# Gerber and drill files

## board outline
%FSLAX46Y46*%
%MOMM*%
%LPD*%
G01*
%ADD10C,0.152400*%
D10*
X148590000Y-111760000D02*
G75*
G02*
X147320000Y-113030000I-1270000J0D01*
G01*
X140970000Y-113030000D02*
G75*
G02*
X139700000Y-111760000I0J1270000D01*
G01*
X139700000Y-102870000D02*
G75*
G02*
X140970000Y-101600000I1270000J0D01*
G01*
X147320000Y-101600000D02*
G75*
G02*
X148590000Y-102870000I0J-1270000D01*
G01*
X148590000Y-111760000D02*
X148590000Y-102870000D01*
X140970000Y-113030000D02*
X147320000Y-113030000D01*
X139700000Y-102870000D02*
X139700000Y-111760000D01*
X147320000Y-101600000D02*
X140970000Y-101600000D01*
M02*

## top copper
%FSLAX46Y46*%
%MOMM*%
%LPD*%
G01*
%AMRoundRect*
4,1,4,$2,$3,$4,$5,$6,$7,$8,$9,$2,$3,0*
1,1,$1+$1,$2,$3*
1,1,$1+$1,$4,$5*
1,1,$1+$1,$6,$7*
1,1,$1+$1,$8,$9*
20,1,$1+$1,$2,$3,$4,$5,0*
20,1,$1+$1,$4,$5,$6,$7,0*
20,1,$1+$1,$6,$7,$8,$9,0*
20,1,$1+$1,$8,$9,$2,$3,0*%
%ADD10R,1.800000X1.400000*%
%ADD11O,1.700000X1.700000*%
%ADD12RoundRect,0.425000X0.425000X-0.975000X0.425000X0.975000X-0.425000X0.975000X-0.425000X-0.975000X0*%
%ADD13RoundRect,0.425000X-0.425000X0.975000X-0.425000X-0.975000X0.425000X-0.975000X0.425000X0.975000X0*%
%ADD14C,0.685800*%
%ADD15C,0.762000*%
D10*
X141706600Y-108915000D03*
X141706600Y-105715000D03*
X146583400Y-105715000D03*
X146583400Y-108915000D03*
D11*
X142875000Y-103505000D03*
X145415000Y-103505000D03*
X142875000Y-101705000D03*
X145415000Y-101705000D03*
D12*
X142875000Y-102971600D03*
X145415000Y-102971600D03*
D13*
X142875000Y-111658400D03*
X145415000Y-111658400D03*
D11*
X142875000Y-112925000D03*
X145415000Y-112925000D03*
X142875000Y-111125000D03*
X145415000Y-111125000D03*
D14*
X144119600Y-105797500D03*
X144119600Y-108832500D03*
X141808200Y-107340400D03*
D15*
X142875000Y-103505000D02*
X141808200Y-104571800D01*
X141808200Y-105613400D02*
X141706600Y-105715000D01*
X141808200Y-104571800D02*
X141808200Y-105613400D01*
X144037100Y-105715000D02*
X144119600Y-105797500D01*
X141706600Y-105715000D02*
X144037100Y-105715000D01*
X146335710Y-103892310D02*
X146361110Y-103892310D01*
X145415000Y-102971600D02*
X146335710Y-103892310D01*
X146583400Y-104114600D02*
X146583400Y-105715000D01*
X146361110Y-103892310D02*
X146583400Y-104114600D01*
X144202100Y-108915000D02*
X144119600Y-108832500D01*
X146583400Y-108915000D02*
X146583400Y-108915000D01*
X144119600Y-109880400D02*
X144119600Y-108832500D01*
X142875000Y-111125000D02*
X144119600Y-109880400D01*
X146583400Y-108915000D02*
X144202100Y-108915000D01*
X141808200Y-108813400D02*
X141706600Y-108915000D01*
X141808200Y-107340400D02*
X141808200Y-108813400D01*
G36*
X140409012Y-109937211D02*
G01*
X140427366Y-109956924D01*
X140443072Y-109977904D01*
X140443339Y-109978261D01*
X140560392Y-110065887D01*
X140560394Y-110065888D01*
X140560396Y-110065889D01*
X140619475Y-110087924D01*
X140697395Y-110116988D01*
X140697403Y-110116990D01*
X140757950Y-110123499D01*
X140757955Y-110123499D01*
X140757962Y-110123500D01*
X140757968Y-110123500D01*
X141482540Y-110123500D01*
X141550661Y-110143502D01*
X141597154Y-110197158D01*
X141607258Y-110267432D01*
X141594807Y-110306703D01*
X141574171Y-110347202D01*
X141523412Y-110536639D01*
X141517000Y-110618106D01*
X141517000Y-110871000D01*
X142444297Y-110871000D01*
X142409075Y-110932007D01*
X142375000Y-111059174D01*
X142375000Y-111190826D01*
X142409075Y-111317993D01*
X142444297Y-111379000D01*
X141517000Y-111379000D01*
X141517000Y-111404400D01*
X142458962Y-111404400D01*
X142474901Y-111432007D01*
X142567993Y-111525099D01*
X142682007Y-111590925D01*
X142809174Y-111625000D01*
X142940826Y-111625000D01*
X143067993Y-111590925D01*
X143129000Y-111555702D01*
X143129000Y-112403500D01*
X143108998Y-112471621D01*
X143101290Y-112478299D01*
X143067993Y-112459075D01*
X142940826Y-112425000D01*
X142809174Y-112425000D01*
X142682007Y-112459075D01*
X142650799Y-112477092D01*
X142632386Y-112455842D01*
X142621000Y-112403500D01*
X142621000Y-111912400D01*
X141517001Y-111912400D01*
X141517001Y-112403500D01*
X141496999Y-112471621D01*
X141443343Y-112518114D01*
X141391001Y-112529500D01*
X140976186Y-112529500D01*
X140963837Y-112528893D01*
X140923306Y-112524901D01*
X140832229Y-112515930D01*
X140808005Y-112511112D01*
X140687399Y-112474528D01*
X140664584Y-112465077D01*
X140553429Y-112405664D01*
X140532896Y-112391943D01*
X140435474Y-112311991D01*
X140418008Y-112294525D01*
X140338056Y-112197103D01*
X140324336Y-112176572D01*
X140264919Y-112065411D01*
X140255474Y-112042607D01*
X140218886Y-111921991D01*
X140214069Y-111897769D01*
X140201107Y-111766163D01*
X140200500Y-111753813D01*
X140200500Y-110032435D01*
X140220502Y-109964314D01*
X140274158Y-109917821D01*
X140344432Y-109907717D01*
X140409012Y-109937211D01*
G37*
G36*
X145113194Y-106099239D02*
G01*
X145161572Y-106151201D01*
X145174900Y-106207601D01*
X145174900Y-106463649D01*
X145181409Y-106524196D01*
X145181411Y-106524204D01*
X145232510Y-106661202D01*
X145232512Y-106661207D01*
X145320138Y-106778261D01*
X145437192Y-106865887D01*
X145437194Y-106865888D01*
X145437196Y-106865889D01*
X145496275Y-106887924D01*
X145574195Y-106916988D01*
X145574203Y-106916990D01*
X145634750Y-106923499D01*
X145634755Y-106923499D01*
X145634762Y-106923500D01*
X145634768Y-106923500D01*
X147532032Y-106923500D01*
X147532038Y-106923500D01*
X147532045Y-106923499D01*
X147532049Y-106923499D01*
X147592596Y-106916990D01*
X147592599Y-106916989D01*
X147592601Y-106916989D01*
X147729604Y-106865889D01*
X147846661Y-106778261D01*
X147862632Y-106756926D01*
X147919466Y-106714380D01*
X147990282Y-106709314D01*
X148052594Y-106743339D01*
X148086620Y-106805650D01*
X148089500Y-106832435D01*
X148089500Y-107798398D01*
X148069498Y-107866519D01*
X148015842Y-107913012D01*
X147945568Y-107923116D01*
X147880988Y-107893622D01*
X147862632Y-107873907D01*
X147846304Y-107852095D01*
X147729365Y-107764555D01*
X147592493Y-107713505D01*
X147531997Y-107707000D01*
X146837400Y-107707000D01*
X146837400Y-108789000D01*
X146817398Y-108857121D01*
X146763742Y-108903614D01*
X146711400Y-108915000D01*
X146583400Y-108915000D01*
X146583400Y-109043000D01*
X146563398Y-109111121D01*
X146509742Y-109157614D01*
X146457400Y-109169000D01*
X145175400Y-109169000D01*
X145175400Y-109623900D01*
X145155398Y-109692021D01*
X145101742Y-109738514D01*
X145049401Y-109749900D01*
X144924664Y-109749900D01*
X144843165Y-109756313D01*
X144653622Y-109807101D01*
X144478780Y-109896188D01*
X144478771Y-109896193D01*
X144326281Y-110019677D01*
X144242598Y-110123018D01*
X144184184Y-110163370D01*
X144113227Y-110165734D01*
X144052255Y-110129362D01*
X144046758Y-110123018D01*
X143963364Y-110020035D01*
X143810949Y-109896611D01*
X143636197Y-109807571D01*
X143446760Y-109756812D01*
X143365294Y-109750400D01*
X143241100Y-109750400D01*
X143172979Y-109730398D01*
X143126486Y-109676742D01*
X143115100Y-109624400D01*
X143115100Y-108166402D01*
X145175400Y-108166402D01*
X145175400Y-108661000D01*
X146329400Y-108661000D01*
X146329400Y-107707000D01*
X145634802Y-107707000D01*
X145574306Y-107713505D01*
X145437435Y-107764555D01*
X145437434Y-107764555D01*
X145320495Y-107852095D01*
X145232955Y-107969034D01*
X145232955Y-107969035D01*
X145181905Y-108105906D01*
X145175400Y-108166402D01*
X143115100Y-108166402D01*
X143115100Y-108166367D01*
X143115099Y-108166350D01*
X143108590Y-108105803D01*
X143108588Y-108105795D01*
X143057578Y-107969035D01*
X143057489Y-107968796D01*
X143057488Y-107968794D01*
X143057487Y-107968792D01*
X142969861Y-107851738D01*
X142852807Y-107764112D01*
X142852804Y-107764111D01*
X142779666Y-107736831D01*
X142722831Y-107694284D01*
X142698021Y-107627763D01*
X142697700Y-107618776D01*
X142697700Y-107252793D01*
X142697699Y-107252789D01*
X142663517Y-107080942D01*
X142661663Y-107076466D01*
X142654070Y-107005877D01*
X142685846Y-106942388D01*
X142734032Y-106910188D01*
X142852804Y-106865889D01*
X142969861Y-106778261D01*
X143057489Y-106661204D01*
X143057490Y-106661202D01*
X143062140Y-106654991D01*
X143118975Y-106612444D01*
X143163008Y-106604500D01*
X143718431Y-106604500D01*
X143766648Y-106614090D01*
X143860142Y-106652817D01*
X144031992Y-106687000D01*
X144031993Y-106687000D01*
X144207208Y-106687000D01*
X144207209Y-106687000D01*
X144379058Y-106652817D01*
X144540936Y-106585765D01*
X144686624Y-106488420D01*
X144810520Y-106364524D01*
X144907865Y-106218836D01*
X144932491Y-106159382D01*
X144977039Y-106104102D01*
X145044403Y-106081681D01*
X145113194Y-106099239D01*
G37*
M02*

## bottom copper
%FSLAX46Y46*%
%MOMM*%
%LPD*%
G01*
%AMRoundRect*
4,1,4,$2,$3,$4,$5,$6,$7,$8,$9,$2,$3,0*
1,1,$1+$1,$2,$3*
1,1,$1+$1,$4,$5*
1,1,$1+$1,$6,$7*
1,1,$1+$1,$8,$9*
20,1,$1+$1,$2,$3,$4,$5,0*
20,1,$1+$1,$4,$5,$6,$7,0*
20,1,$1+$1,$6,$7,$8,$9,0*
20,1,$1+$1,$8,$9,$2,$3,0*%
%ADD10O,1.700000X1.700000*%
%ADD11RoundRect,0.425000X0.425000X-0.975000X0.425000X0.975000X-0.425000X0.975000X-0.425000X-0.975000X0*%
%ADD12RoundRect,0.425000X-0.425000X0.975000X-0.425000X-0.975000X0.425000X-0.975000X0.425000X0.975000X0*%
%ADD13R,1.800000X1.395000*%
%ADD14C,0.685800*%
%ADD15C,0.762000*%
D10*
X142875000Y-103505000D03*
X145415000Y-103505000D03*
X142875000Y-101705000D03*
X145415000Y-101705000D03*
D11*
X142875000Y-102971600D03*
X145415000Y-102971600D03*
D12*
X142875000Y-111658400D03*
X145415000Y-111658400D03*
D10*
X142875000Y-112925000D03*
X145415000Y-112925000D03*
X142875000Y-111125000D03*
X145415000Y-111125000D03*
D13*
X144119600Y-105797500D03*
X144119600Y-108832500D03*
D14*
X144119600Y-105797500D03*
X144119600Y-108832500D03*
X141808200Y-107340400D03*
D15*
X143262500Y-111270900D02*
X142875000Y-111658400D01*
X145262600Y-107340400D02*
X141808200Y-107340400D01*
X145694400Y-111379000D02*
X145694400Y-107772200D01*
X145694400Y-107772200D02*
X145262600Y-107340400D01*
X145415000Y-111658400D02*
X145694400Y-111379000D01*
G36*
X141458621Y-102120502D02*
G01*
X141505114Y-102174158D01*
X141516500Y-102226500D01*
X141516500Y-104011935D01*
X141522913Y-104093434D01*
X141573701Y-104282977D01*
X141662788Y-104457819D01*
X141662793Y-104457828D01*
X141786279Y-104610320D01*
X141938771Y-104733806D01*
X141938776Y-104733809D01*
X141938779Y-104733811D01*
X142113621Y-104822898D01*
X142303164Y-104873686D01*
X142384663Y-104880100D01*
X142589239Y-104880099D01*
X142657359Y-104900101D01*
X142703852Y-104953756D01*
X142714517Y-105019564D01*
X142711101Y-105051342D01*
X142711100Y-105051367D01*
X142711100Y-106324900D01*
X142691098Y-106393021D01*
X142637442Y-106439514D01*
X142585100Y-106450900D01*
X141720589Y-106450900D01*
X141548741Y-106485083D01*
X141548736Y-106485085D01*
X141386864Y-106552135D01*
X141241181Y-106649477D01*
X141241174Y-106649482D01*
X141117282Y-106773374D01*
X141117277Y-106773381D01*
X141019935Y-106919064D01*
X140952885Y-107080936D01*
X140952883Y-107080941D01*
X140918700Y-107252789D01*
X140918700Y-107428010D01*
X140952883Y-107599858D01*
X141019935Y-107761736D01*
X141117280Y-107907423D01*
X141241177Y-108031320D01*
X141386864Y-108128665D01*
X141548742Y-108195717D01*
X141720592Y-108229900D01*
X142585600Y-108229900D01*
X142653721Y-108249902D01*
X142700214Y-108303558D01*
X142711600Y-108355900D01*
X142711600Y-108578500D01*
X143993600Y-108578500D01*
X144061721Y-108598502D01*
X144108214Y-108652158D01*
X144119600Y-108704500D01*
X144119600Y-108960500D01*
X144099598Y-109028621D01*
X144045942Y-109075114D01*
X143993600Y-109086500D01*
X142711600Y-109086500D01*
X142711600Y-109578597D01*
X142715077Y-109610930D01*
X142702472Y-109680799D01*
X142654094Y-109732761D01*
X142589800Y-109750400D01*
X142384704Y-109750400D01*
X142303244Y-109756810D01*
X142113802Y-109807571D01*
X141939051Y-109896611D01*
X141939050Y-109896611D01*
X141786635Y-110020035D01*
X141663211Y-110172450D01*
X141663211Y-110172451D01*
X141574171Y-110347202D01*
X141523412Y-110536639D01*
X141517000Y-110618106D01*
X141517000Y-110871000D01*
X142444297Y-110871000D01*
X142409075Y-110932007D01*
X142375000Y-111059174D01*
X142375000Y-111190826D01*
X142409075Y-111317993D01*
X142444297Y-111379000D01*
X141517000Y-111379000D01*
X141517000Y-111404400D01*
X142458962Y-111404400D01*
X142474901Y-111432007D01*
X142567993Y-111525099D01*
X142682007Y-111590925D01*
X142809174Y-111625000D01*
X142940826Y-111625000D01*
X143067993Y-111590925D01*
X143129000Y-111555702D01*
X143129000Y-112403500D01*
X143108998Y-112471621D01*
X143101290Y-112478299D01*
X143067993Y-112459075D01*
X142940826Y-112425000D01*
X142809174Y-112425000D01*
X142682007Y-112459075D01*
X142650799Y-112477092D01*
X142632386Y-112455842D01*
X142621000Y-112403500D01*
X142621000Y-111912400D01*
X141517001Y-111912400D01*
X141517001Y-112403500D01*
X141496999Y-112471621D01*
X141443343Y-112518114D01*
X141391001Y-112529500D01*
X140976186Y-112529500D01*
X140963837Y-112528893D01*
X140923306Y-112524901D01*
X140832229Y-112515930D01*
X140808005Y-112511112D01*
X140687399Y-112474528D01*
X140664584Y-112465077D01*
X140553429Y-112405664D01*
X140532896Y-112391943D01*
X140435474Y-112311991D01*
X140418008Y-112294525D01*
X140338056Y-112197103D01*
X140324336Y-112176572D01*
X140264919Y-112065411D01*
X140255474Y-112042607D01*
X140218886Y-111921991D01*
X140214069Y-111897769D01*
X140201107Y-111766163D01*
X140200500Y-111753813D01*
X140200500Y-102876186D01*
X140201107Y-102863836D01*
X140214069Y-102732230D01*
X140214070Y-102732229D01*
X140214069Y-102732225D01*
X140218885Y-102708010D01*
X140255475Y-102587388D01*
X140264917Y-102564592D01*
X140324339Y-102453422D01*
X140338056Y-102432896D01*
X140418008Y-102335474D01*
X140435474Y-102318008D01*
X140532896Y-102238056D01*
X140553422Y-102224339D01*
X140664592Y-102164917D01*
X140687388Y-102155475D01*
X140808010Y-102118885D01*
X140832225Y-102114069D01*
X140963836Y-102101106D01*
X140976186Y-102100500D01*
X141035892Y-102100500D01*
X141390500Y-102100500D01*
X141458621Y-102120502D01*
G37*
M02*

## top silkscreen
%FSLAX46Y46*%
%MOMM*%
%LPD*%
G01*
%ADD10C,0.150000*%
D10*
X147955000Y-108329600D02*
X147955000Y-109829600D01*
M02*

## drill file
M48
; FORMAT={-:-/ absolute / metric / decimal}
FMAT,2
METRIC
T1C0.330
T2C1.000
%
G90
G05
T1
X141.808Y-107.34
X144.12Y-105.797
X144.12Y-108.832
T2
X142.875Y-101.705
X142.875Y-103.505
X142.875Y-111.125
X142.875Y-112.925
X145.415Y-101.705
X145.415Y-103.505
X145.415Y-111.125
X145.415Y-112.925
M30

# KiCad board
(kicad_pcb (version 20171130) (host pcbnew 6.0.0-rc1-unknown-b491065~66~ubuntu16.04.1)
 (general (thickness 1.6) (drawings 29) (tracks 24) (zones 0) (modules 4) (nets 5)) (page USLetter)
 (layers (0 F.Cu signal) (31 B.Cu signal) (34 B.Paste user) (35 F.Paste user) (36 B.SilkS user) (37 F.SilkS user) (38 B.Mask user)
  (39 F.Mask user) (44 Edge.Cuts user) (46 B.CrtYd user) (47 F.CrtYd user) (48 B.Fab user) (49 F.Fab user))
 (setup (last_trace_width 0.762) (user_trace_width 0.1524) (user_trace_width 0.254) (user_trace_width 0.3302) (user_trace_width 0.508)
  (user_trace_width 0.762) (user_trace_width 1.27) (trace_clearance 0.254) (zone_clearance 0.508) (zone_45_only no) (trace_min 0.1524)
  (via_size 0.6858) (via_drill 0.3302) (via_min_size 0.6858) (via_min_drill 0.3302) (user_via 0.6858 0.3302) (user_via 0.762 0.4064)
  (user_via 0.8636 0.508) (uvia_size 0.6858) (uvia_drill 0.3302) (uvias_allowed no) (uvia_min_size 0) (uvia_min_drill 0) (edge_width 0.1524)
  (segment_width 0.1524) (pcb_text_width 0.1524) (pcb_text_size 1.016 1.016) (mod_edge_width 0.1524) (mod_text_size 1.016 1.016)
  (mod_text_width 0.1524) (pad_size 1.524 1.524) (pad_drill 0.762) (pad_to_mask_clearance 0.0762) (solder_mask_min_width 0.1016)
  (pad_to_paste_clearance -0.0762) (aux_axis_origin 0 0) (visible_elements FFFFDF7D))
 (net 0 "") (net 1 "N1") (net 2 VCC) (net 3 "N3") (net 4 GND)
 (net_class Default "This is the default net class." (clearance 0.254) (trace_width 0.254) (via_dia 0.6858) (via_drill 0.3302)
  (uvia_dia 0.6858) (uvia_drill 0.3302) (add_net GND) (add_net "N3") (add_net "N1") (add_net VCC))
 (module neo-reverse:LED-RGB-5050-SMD (layer F.Cu) (at 144.145 107.315)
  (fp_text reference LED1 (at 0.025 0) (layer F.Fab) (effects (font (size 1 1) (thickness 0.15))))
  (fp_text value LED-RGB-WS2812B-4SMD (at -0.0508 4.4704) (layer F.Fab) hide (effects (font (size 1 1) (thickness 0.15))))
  (fp_line (start 3.81 1.0146) (end 3.81 2.5146) (layer F.SilkS) (width 0.15))
  (pad 4 smd rect (at -2.4384 1.6) (size 1.8 1.4) (layers F.Cu F.Paste F.Mask) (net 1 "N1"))
  (pad 3 smd rect (at -2.4384 -1.6) (size 1.8 1.4) (layers F.Cu F.Paste F.Mask) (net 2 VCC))
  (pad 2 smd rect (at 2.4384 -1.6) (size 1.8 1.4) (layers F.Cu F.Paste F.Mask) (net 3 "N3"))
  (pad 1 smd rect (at 2.4384 1.6) (size 1.8 1.4) (layers F.Cu F.Paste F.Mask) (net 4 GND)))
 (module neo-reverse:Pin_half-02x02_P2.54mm (layer F.Cu) (at 142.875 103.505 90)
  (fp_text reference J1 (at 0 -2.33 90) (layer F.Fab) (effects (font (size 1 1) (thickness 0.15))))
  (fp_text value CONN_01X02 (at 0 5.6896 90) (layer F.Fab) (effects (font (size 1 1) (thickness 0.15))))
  (pad 1 thru_hole oval (at 0 0 90) (size 1.7 1.7) (drill 1) (layers *.Cu *.Mask) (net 2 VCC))
  (pad 2 thru_hole oval (at 0 2.54 90) (size 1.7 1.7) (drill 1) (layers *.Cu *.Mask) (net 3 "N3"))
  (pad 1 thru_hole oval (at 1.8 0 90) (size 1.7 1.7) (drill 1) (layers *.Cu *.Mask) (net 2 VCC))
  (pad 2 thru_hole oval (at 1.8 2.54 90) (size 1.7 1.7) (drill 1) (layers *.Cu *.Mask) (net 3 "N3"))
  (pad 1 smd roundrect (at 0.5334 0 90) (size 2.8 1.7) (layers F.Cu F.Mask) (roundrect_rratio 0.25) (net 2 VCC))
  (pad 1 smd roundrect (at 0.5334 0 90) (size 2.8 1.7) (layers B.Cu B.Mask) (roundrect_rratio 0.25) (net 2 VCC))
  (pad 2 smd roundrect (at 0.5334 2.54 90) (size 2.8 1.7) (layers F.Cu F.Mask) (roundrect_rratio 0.25) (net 3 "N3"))
  (pad 2 smd roundrect (at 0.5334 2.54 90) (size 2.8 1.7) (layers B.Cu B.Mask) (roundrect_rratio 0.25) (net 3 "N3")))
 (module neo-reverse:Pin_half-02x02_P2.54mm (layer F.Cu) (at 145.415 111.125 270)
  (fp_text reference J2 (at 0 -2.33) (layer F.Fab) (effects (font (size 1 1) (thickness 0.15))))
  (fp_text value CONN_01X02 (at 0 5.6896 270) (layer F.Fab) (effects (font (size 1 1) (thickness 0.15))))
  (pad 2 smd roundrect (at 0.5334 2.54 270) (size 2.8 1.7) (layers B.Cu B.Mask) (roundrect_rratio 0.25) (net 4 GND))
  (pad 2 smd roundrect (at 0.5334 2.54 270) (size 2.8 1.7) (layers F.Cu F.Mask) (roundrect_rratio 0.25) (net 4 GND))
  (pad 1 smd roundrect (at 0.5334 0 270) (size 2.8 1.7) (layers B.Cu B.Mask) (roundrect_rratio 0.25) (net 1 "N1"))
  (pad 1 smd roundrect (at 0.5334 0 270) (size 2.8 1.7) (layers F.Cu F.Mask) (roundrect_rratio 0.25) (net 1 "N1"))
  (pad 2 thru_hole oval (at 1.8 2.54 270) (size 1.7 1.7) (drill 1) (layers *.Cu *.Mask) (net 4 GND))
  (pad 1 thru_hole oval (at 1.8 0 270) (size 1.7 1.7) (drill 1) (layers *.Cu *.Mask) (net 1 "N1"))
  (pad 2 thru_hole oval (at 0 2.54 270) (size 1.7 1.7) (drill 1) (layers *.Cu *.Mask) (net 4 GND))
  (pad 1 thru_hole oval (at 0 0 270) (size 1.7 1.7) (drill 1) (layers *.Cu *.Mask) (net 1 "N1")))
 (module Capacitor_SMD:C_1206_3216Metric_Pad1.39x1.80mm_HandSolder (layer B.Cu) (at 144.1196 107.315 270)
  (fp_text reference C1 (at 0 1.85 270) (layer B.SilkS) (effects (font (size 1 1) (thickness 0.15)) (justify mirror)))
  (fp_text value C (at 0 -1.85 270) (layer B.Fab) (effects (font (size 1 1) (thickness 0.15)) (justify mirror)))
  (pad 1 smd rect (at -1.5175 0 270) (size 1.395 1.8) (layers B.Cu B.Paste B.Mask) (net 2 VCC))
  (pad 2 smd rect (at 1.5175 0 270) (size 1.395 1.8) (layers B.Cu B.Paste B.Mask) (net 4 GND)))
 (gr_arc (start 147.32 111.76) (end 147.32 113.03) (angle -90) (layer Edge.Cuts) (width 0.1524))
 (gr_arc (start 140.97 111.76) (end 139.7 111.76) (angle -90) (layer Edge.Cuts) (width 0.1524))
 (gr_arc (start 140.97 102.87) (end 140.97 101.6) (angle -90) (layer Edge.Cuts) (width 0.1524))
 (gr_arc (start 147.32 102.87) (end 148.59 102.87) (angle -90) (layer Edge.Cuts) (width 0.1524))
 (gr_line (start 148.59 111.76) (end 148.59 102.87) (layer Edge.Cuts) (width 0.1524))
 (gr_line (start 140.97 113.03) (end 147.32 113.03) (layer Edge.Cuts) (width 0.1524))
 (gr_line (start 139.7 102.87) (end 139.7 111.76) (layer Edge.Cuts) (width 0.1524))
 (gr_line (start 147.32 101.6) (end 140.97 101.6) (layer Edge.Cuts) (width 0.1524))
 (segment (start 142.875 103.505) (end 141.8082 104.5718) (width 0.762) (layer F.Cu) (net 2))
 (segment (start 141.8082 105.6134) (end 141.7066 105.715) (width 0.762) (layer F.Cu) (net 2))
 (segment (start 141.8082 104.5718) (end 141.8082 105.6134) (width 0.762) (layer F.Cu) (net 2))
 (segment (start 144.0371 105.715) (end 144.1196 105.7975) (width 0.762) (layer F.Cu) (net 2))
 (via (at 144.1196 105.7975) (size 0.6858) (drill 0.3302) (layers F.Cu B.Cu) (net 2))
 (segment (start 141.7066 105.715) (end 144.0371 105.715) (width 0.762) (layer F.Cu) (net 2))
 (segment (start 146.33571 103.89231) (end 146.36111 103.89231) (width 0.762) (layer F.Cu) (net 3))
 (segment (start 145.415 102.9716) (end 146.33571 103.89231) (width 0.762) (layer F.Cu) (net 3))
 (segment (start 146.5834 104.1146) (end 146.5834 105.715) (width 0.762) (layer F.Cu) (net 3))
 (segment (start 146.36111 103.89231) (end 146.5834 104.1146) (width 0.762) (layer F.Cu) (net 3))
 (segment (start 143.2625 111.2709) (end 142.875 111.6584) (width 0.762) (layer B.Cu) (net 4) (status 30))
 (via (at 144.1196 108.8325) (size 0.6858) (drill 0.3302) (layers F.Cu B.Cu) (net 4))
 (segment (start 144.2021 108.915) (end 144.1196 108.8325) (width 0.762) (layer F.Cu) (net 4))
 (segment (start 146.5834 108.915) (end 146.5834 108.915) (width 0.762) (layer F.Cu) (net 4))
 (segment (start 144.1196 109.8804) (end 144.1196 108.8325) (width 0.762) (layer F.Cu) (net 4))
 (segment (start 142.875 111.125) (end 144.1196 109.8804) (width 0.762) (layer F.Cu) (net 4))
 (segment (start 146.5834 108.915) (end 144.2021 108.915) (width 0.762) (layer F.Cu) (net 4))
 (via (at 141.8082 107.3404) (size 0.6858) (drill 0.3302) (layers F.Cu B.Cu) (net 1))
 (segment (start 141.8082 108.8134) (end 141.7066 108.915) (width 0.762) (layer F.Cu) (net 1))
 (segment (start 141.8082 107.3404) (end 141.8082 108.8134) (width 0.762) (layer F.Cu) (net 1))
 (segment (start 145.2626 107.3404) (end 141.8082 107.3404) (width 0.762) (layer B.Cu) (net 1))
 (segment (start 145.6944 111.379) (end 145.6944 107.7722) (width 0.762) (layer B.Cu) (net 1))
 (segment (start 145.6944 107.7722) (end 145.2626 107.3404) (width 0.762) (layer B.Cu) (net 1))
 (segment (start 145.415 111.6584) (end 145.6944 111.379) (width 0.762) (layer B.Cu) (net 1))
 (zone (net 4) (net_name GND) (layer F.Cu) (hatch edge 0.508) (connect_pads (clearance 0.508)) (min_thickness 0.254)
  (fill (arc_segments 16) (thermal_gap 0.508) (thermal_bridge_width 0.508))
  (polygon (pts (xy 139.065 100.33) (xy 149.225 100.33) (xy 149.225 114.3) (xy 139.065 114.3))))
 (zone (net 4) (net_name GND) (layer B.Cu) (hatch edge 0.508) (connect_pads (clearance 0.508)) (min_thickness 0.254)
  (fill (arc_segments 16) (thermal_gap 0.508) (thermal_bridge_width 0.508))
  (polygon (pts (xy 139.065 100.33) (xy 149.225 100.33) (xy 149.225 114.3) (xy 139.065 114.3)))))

